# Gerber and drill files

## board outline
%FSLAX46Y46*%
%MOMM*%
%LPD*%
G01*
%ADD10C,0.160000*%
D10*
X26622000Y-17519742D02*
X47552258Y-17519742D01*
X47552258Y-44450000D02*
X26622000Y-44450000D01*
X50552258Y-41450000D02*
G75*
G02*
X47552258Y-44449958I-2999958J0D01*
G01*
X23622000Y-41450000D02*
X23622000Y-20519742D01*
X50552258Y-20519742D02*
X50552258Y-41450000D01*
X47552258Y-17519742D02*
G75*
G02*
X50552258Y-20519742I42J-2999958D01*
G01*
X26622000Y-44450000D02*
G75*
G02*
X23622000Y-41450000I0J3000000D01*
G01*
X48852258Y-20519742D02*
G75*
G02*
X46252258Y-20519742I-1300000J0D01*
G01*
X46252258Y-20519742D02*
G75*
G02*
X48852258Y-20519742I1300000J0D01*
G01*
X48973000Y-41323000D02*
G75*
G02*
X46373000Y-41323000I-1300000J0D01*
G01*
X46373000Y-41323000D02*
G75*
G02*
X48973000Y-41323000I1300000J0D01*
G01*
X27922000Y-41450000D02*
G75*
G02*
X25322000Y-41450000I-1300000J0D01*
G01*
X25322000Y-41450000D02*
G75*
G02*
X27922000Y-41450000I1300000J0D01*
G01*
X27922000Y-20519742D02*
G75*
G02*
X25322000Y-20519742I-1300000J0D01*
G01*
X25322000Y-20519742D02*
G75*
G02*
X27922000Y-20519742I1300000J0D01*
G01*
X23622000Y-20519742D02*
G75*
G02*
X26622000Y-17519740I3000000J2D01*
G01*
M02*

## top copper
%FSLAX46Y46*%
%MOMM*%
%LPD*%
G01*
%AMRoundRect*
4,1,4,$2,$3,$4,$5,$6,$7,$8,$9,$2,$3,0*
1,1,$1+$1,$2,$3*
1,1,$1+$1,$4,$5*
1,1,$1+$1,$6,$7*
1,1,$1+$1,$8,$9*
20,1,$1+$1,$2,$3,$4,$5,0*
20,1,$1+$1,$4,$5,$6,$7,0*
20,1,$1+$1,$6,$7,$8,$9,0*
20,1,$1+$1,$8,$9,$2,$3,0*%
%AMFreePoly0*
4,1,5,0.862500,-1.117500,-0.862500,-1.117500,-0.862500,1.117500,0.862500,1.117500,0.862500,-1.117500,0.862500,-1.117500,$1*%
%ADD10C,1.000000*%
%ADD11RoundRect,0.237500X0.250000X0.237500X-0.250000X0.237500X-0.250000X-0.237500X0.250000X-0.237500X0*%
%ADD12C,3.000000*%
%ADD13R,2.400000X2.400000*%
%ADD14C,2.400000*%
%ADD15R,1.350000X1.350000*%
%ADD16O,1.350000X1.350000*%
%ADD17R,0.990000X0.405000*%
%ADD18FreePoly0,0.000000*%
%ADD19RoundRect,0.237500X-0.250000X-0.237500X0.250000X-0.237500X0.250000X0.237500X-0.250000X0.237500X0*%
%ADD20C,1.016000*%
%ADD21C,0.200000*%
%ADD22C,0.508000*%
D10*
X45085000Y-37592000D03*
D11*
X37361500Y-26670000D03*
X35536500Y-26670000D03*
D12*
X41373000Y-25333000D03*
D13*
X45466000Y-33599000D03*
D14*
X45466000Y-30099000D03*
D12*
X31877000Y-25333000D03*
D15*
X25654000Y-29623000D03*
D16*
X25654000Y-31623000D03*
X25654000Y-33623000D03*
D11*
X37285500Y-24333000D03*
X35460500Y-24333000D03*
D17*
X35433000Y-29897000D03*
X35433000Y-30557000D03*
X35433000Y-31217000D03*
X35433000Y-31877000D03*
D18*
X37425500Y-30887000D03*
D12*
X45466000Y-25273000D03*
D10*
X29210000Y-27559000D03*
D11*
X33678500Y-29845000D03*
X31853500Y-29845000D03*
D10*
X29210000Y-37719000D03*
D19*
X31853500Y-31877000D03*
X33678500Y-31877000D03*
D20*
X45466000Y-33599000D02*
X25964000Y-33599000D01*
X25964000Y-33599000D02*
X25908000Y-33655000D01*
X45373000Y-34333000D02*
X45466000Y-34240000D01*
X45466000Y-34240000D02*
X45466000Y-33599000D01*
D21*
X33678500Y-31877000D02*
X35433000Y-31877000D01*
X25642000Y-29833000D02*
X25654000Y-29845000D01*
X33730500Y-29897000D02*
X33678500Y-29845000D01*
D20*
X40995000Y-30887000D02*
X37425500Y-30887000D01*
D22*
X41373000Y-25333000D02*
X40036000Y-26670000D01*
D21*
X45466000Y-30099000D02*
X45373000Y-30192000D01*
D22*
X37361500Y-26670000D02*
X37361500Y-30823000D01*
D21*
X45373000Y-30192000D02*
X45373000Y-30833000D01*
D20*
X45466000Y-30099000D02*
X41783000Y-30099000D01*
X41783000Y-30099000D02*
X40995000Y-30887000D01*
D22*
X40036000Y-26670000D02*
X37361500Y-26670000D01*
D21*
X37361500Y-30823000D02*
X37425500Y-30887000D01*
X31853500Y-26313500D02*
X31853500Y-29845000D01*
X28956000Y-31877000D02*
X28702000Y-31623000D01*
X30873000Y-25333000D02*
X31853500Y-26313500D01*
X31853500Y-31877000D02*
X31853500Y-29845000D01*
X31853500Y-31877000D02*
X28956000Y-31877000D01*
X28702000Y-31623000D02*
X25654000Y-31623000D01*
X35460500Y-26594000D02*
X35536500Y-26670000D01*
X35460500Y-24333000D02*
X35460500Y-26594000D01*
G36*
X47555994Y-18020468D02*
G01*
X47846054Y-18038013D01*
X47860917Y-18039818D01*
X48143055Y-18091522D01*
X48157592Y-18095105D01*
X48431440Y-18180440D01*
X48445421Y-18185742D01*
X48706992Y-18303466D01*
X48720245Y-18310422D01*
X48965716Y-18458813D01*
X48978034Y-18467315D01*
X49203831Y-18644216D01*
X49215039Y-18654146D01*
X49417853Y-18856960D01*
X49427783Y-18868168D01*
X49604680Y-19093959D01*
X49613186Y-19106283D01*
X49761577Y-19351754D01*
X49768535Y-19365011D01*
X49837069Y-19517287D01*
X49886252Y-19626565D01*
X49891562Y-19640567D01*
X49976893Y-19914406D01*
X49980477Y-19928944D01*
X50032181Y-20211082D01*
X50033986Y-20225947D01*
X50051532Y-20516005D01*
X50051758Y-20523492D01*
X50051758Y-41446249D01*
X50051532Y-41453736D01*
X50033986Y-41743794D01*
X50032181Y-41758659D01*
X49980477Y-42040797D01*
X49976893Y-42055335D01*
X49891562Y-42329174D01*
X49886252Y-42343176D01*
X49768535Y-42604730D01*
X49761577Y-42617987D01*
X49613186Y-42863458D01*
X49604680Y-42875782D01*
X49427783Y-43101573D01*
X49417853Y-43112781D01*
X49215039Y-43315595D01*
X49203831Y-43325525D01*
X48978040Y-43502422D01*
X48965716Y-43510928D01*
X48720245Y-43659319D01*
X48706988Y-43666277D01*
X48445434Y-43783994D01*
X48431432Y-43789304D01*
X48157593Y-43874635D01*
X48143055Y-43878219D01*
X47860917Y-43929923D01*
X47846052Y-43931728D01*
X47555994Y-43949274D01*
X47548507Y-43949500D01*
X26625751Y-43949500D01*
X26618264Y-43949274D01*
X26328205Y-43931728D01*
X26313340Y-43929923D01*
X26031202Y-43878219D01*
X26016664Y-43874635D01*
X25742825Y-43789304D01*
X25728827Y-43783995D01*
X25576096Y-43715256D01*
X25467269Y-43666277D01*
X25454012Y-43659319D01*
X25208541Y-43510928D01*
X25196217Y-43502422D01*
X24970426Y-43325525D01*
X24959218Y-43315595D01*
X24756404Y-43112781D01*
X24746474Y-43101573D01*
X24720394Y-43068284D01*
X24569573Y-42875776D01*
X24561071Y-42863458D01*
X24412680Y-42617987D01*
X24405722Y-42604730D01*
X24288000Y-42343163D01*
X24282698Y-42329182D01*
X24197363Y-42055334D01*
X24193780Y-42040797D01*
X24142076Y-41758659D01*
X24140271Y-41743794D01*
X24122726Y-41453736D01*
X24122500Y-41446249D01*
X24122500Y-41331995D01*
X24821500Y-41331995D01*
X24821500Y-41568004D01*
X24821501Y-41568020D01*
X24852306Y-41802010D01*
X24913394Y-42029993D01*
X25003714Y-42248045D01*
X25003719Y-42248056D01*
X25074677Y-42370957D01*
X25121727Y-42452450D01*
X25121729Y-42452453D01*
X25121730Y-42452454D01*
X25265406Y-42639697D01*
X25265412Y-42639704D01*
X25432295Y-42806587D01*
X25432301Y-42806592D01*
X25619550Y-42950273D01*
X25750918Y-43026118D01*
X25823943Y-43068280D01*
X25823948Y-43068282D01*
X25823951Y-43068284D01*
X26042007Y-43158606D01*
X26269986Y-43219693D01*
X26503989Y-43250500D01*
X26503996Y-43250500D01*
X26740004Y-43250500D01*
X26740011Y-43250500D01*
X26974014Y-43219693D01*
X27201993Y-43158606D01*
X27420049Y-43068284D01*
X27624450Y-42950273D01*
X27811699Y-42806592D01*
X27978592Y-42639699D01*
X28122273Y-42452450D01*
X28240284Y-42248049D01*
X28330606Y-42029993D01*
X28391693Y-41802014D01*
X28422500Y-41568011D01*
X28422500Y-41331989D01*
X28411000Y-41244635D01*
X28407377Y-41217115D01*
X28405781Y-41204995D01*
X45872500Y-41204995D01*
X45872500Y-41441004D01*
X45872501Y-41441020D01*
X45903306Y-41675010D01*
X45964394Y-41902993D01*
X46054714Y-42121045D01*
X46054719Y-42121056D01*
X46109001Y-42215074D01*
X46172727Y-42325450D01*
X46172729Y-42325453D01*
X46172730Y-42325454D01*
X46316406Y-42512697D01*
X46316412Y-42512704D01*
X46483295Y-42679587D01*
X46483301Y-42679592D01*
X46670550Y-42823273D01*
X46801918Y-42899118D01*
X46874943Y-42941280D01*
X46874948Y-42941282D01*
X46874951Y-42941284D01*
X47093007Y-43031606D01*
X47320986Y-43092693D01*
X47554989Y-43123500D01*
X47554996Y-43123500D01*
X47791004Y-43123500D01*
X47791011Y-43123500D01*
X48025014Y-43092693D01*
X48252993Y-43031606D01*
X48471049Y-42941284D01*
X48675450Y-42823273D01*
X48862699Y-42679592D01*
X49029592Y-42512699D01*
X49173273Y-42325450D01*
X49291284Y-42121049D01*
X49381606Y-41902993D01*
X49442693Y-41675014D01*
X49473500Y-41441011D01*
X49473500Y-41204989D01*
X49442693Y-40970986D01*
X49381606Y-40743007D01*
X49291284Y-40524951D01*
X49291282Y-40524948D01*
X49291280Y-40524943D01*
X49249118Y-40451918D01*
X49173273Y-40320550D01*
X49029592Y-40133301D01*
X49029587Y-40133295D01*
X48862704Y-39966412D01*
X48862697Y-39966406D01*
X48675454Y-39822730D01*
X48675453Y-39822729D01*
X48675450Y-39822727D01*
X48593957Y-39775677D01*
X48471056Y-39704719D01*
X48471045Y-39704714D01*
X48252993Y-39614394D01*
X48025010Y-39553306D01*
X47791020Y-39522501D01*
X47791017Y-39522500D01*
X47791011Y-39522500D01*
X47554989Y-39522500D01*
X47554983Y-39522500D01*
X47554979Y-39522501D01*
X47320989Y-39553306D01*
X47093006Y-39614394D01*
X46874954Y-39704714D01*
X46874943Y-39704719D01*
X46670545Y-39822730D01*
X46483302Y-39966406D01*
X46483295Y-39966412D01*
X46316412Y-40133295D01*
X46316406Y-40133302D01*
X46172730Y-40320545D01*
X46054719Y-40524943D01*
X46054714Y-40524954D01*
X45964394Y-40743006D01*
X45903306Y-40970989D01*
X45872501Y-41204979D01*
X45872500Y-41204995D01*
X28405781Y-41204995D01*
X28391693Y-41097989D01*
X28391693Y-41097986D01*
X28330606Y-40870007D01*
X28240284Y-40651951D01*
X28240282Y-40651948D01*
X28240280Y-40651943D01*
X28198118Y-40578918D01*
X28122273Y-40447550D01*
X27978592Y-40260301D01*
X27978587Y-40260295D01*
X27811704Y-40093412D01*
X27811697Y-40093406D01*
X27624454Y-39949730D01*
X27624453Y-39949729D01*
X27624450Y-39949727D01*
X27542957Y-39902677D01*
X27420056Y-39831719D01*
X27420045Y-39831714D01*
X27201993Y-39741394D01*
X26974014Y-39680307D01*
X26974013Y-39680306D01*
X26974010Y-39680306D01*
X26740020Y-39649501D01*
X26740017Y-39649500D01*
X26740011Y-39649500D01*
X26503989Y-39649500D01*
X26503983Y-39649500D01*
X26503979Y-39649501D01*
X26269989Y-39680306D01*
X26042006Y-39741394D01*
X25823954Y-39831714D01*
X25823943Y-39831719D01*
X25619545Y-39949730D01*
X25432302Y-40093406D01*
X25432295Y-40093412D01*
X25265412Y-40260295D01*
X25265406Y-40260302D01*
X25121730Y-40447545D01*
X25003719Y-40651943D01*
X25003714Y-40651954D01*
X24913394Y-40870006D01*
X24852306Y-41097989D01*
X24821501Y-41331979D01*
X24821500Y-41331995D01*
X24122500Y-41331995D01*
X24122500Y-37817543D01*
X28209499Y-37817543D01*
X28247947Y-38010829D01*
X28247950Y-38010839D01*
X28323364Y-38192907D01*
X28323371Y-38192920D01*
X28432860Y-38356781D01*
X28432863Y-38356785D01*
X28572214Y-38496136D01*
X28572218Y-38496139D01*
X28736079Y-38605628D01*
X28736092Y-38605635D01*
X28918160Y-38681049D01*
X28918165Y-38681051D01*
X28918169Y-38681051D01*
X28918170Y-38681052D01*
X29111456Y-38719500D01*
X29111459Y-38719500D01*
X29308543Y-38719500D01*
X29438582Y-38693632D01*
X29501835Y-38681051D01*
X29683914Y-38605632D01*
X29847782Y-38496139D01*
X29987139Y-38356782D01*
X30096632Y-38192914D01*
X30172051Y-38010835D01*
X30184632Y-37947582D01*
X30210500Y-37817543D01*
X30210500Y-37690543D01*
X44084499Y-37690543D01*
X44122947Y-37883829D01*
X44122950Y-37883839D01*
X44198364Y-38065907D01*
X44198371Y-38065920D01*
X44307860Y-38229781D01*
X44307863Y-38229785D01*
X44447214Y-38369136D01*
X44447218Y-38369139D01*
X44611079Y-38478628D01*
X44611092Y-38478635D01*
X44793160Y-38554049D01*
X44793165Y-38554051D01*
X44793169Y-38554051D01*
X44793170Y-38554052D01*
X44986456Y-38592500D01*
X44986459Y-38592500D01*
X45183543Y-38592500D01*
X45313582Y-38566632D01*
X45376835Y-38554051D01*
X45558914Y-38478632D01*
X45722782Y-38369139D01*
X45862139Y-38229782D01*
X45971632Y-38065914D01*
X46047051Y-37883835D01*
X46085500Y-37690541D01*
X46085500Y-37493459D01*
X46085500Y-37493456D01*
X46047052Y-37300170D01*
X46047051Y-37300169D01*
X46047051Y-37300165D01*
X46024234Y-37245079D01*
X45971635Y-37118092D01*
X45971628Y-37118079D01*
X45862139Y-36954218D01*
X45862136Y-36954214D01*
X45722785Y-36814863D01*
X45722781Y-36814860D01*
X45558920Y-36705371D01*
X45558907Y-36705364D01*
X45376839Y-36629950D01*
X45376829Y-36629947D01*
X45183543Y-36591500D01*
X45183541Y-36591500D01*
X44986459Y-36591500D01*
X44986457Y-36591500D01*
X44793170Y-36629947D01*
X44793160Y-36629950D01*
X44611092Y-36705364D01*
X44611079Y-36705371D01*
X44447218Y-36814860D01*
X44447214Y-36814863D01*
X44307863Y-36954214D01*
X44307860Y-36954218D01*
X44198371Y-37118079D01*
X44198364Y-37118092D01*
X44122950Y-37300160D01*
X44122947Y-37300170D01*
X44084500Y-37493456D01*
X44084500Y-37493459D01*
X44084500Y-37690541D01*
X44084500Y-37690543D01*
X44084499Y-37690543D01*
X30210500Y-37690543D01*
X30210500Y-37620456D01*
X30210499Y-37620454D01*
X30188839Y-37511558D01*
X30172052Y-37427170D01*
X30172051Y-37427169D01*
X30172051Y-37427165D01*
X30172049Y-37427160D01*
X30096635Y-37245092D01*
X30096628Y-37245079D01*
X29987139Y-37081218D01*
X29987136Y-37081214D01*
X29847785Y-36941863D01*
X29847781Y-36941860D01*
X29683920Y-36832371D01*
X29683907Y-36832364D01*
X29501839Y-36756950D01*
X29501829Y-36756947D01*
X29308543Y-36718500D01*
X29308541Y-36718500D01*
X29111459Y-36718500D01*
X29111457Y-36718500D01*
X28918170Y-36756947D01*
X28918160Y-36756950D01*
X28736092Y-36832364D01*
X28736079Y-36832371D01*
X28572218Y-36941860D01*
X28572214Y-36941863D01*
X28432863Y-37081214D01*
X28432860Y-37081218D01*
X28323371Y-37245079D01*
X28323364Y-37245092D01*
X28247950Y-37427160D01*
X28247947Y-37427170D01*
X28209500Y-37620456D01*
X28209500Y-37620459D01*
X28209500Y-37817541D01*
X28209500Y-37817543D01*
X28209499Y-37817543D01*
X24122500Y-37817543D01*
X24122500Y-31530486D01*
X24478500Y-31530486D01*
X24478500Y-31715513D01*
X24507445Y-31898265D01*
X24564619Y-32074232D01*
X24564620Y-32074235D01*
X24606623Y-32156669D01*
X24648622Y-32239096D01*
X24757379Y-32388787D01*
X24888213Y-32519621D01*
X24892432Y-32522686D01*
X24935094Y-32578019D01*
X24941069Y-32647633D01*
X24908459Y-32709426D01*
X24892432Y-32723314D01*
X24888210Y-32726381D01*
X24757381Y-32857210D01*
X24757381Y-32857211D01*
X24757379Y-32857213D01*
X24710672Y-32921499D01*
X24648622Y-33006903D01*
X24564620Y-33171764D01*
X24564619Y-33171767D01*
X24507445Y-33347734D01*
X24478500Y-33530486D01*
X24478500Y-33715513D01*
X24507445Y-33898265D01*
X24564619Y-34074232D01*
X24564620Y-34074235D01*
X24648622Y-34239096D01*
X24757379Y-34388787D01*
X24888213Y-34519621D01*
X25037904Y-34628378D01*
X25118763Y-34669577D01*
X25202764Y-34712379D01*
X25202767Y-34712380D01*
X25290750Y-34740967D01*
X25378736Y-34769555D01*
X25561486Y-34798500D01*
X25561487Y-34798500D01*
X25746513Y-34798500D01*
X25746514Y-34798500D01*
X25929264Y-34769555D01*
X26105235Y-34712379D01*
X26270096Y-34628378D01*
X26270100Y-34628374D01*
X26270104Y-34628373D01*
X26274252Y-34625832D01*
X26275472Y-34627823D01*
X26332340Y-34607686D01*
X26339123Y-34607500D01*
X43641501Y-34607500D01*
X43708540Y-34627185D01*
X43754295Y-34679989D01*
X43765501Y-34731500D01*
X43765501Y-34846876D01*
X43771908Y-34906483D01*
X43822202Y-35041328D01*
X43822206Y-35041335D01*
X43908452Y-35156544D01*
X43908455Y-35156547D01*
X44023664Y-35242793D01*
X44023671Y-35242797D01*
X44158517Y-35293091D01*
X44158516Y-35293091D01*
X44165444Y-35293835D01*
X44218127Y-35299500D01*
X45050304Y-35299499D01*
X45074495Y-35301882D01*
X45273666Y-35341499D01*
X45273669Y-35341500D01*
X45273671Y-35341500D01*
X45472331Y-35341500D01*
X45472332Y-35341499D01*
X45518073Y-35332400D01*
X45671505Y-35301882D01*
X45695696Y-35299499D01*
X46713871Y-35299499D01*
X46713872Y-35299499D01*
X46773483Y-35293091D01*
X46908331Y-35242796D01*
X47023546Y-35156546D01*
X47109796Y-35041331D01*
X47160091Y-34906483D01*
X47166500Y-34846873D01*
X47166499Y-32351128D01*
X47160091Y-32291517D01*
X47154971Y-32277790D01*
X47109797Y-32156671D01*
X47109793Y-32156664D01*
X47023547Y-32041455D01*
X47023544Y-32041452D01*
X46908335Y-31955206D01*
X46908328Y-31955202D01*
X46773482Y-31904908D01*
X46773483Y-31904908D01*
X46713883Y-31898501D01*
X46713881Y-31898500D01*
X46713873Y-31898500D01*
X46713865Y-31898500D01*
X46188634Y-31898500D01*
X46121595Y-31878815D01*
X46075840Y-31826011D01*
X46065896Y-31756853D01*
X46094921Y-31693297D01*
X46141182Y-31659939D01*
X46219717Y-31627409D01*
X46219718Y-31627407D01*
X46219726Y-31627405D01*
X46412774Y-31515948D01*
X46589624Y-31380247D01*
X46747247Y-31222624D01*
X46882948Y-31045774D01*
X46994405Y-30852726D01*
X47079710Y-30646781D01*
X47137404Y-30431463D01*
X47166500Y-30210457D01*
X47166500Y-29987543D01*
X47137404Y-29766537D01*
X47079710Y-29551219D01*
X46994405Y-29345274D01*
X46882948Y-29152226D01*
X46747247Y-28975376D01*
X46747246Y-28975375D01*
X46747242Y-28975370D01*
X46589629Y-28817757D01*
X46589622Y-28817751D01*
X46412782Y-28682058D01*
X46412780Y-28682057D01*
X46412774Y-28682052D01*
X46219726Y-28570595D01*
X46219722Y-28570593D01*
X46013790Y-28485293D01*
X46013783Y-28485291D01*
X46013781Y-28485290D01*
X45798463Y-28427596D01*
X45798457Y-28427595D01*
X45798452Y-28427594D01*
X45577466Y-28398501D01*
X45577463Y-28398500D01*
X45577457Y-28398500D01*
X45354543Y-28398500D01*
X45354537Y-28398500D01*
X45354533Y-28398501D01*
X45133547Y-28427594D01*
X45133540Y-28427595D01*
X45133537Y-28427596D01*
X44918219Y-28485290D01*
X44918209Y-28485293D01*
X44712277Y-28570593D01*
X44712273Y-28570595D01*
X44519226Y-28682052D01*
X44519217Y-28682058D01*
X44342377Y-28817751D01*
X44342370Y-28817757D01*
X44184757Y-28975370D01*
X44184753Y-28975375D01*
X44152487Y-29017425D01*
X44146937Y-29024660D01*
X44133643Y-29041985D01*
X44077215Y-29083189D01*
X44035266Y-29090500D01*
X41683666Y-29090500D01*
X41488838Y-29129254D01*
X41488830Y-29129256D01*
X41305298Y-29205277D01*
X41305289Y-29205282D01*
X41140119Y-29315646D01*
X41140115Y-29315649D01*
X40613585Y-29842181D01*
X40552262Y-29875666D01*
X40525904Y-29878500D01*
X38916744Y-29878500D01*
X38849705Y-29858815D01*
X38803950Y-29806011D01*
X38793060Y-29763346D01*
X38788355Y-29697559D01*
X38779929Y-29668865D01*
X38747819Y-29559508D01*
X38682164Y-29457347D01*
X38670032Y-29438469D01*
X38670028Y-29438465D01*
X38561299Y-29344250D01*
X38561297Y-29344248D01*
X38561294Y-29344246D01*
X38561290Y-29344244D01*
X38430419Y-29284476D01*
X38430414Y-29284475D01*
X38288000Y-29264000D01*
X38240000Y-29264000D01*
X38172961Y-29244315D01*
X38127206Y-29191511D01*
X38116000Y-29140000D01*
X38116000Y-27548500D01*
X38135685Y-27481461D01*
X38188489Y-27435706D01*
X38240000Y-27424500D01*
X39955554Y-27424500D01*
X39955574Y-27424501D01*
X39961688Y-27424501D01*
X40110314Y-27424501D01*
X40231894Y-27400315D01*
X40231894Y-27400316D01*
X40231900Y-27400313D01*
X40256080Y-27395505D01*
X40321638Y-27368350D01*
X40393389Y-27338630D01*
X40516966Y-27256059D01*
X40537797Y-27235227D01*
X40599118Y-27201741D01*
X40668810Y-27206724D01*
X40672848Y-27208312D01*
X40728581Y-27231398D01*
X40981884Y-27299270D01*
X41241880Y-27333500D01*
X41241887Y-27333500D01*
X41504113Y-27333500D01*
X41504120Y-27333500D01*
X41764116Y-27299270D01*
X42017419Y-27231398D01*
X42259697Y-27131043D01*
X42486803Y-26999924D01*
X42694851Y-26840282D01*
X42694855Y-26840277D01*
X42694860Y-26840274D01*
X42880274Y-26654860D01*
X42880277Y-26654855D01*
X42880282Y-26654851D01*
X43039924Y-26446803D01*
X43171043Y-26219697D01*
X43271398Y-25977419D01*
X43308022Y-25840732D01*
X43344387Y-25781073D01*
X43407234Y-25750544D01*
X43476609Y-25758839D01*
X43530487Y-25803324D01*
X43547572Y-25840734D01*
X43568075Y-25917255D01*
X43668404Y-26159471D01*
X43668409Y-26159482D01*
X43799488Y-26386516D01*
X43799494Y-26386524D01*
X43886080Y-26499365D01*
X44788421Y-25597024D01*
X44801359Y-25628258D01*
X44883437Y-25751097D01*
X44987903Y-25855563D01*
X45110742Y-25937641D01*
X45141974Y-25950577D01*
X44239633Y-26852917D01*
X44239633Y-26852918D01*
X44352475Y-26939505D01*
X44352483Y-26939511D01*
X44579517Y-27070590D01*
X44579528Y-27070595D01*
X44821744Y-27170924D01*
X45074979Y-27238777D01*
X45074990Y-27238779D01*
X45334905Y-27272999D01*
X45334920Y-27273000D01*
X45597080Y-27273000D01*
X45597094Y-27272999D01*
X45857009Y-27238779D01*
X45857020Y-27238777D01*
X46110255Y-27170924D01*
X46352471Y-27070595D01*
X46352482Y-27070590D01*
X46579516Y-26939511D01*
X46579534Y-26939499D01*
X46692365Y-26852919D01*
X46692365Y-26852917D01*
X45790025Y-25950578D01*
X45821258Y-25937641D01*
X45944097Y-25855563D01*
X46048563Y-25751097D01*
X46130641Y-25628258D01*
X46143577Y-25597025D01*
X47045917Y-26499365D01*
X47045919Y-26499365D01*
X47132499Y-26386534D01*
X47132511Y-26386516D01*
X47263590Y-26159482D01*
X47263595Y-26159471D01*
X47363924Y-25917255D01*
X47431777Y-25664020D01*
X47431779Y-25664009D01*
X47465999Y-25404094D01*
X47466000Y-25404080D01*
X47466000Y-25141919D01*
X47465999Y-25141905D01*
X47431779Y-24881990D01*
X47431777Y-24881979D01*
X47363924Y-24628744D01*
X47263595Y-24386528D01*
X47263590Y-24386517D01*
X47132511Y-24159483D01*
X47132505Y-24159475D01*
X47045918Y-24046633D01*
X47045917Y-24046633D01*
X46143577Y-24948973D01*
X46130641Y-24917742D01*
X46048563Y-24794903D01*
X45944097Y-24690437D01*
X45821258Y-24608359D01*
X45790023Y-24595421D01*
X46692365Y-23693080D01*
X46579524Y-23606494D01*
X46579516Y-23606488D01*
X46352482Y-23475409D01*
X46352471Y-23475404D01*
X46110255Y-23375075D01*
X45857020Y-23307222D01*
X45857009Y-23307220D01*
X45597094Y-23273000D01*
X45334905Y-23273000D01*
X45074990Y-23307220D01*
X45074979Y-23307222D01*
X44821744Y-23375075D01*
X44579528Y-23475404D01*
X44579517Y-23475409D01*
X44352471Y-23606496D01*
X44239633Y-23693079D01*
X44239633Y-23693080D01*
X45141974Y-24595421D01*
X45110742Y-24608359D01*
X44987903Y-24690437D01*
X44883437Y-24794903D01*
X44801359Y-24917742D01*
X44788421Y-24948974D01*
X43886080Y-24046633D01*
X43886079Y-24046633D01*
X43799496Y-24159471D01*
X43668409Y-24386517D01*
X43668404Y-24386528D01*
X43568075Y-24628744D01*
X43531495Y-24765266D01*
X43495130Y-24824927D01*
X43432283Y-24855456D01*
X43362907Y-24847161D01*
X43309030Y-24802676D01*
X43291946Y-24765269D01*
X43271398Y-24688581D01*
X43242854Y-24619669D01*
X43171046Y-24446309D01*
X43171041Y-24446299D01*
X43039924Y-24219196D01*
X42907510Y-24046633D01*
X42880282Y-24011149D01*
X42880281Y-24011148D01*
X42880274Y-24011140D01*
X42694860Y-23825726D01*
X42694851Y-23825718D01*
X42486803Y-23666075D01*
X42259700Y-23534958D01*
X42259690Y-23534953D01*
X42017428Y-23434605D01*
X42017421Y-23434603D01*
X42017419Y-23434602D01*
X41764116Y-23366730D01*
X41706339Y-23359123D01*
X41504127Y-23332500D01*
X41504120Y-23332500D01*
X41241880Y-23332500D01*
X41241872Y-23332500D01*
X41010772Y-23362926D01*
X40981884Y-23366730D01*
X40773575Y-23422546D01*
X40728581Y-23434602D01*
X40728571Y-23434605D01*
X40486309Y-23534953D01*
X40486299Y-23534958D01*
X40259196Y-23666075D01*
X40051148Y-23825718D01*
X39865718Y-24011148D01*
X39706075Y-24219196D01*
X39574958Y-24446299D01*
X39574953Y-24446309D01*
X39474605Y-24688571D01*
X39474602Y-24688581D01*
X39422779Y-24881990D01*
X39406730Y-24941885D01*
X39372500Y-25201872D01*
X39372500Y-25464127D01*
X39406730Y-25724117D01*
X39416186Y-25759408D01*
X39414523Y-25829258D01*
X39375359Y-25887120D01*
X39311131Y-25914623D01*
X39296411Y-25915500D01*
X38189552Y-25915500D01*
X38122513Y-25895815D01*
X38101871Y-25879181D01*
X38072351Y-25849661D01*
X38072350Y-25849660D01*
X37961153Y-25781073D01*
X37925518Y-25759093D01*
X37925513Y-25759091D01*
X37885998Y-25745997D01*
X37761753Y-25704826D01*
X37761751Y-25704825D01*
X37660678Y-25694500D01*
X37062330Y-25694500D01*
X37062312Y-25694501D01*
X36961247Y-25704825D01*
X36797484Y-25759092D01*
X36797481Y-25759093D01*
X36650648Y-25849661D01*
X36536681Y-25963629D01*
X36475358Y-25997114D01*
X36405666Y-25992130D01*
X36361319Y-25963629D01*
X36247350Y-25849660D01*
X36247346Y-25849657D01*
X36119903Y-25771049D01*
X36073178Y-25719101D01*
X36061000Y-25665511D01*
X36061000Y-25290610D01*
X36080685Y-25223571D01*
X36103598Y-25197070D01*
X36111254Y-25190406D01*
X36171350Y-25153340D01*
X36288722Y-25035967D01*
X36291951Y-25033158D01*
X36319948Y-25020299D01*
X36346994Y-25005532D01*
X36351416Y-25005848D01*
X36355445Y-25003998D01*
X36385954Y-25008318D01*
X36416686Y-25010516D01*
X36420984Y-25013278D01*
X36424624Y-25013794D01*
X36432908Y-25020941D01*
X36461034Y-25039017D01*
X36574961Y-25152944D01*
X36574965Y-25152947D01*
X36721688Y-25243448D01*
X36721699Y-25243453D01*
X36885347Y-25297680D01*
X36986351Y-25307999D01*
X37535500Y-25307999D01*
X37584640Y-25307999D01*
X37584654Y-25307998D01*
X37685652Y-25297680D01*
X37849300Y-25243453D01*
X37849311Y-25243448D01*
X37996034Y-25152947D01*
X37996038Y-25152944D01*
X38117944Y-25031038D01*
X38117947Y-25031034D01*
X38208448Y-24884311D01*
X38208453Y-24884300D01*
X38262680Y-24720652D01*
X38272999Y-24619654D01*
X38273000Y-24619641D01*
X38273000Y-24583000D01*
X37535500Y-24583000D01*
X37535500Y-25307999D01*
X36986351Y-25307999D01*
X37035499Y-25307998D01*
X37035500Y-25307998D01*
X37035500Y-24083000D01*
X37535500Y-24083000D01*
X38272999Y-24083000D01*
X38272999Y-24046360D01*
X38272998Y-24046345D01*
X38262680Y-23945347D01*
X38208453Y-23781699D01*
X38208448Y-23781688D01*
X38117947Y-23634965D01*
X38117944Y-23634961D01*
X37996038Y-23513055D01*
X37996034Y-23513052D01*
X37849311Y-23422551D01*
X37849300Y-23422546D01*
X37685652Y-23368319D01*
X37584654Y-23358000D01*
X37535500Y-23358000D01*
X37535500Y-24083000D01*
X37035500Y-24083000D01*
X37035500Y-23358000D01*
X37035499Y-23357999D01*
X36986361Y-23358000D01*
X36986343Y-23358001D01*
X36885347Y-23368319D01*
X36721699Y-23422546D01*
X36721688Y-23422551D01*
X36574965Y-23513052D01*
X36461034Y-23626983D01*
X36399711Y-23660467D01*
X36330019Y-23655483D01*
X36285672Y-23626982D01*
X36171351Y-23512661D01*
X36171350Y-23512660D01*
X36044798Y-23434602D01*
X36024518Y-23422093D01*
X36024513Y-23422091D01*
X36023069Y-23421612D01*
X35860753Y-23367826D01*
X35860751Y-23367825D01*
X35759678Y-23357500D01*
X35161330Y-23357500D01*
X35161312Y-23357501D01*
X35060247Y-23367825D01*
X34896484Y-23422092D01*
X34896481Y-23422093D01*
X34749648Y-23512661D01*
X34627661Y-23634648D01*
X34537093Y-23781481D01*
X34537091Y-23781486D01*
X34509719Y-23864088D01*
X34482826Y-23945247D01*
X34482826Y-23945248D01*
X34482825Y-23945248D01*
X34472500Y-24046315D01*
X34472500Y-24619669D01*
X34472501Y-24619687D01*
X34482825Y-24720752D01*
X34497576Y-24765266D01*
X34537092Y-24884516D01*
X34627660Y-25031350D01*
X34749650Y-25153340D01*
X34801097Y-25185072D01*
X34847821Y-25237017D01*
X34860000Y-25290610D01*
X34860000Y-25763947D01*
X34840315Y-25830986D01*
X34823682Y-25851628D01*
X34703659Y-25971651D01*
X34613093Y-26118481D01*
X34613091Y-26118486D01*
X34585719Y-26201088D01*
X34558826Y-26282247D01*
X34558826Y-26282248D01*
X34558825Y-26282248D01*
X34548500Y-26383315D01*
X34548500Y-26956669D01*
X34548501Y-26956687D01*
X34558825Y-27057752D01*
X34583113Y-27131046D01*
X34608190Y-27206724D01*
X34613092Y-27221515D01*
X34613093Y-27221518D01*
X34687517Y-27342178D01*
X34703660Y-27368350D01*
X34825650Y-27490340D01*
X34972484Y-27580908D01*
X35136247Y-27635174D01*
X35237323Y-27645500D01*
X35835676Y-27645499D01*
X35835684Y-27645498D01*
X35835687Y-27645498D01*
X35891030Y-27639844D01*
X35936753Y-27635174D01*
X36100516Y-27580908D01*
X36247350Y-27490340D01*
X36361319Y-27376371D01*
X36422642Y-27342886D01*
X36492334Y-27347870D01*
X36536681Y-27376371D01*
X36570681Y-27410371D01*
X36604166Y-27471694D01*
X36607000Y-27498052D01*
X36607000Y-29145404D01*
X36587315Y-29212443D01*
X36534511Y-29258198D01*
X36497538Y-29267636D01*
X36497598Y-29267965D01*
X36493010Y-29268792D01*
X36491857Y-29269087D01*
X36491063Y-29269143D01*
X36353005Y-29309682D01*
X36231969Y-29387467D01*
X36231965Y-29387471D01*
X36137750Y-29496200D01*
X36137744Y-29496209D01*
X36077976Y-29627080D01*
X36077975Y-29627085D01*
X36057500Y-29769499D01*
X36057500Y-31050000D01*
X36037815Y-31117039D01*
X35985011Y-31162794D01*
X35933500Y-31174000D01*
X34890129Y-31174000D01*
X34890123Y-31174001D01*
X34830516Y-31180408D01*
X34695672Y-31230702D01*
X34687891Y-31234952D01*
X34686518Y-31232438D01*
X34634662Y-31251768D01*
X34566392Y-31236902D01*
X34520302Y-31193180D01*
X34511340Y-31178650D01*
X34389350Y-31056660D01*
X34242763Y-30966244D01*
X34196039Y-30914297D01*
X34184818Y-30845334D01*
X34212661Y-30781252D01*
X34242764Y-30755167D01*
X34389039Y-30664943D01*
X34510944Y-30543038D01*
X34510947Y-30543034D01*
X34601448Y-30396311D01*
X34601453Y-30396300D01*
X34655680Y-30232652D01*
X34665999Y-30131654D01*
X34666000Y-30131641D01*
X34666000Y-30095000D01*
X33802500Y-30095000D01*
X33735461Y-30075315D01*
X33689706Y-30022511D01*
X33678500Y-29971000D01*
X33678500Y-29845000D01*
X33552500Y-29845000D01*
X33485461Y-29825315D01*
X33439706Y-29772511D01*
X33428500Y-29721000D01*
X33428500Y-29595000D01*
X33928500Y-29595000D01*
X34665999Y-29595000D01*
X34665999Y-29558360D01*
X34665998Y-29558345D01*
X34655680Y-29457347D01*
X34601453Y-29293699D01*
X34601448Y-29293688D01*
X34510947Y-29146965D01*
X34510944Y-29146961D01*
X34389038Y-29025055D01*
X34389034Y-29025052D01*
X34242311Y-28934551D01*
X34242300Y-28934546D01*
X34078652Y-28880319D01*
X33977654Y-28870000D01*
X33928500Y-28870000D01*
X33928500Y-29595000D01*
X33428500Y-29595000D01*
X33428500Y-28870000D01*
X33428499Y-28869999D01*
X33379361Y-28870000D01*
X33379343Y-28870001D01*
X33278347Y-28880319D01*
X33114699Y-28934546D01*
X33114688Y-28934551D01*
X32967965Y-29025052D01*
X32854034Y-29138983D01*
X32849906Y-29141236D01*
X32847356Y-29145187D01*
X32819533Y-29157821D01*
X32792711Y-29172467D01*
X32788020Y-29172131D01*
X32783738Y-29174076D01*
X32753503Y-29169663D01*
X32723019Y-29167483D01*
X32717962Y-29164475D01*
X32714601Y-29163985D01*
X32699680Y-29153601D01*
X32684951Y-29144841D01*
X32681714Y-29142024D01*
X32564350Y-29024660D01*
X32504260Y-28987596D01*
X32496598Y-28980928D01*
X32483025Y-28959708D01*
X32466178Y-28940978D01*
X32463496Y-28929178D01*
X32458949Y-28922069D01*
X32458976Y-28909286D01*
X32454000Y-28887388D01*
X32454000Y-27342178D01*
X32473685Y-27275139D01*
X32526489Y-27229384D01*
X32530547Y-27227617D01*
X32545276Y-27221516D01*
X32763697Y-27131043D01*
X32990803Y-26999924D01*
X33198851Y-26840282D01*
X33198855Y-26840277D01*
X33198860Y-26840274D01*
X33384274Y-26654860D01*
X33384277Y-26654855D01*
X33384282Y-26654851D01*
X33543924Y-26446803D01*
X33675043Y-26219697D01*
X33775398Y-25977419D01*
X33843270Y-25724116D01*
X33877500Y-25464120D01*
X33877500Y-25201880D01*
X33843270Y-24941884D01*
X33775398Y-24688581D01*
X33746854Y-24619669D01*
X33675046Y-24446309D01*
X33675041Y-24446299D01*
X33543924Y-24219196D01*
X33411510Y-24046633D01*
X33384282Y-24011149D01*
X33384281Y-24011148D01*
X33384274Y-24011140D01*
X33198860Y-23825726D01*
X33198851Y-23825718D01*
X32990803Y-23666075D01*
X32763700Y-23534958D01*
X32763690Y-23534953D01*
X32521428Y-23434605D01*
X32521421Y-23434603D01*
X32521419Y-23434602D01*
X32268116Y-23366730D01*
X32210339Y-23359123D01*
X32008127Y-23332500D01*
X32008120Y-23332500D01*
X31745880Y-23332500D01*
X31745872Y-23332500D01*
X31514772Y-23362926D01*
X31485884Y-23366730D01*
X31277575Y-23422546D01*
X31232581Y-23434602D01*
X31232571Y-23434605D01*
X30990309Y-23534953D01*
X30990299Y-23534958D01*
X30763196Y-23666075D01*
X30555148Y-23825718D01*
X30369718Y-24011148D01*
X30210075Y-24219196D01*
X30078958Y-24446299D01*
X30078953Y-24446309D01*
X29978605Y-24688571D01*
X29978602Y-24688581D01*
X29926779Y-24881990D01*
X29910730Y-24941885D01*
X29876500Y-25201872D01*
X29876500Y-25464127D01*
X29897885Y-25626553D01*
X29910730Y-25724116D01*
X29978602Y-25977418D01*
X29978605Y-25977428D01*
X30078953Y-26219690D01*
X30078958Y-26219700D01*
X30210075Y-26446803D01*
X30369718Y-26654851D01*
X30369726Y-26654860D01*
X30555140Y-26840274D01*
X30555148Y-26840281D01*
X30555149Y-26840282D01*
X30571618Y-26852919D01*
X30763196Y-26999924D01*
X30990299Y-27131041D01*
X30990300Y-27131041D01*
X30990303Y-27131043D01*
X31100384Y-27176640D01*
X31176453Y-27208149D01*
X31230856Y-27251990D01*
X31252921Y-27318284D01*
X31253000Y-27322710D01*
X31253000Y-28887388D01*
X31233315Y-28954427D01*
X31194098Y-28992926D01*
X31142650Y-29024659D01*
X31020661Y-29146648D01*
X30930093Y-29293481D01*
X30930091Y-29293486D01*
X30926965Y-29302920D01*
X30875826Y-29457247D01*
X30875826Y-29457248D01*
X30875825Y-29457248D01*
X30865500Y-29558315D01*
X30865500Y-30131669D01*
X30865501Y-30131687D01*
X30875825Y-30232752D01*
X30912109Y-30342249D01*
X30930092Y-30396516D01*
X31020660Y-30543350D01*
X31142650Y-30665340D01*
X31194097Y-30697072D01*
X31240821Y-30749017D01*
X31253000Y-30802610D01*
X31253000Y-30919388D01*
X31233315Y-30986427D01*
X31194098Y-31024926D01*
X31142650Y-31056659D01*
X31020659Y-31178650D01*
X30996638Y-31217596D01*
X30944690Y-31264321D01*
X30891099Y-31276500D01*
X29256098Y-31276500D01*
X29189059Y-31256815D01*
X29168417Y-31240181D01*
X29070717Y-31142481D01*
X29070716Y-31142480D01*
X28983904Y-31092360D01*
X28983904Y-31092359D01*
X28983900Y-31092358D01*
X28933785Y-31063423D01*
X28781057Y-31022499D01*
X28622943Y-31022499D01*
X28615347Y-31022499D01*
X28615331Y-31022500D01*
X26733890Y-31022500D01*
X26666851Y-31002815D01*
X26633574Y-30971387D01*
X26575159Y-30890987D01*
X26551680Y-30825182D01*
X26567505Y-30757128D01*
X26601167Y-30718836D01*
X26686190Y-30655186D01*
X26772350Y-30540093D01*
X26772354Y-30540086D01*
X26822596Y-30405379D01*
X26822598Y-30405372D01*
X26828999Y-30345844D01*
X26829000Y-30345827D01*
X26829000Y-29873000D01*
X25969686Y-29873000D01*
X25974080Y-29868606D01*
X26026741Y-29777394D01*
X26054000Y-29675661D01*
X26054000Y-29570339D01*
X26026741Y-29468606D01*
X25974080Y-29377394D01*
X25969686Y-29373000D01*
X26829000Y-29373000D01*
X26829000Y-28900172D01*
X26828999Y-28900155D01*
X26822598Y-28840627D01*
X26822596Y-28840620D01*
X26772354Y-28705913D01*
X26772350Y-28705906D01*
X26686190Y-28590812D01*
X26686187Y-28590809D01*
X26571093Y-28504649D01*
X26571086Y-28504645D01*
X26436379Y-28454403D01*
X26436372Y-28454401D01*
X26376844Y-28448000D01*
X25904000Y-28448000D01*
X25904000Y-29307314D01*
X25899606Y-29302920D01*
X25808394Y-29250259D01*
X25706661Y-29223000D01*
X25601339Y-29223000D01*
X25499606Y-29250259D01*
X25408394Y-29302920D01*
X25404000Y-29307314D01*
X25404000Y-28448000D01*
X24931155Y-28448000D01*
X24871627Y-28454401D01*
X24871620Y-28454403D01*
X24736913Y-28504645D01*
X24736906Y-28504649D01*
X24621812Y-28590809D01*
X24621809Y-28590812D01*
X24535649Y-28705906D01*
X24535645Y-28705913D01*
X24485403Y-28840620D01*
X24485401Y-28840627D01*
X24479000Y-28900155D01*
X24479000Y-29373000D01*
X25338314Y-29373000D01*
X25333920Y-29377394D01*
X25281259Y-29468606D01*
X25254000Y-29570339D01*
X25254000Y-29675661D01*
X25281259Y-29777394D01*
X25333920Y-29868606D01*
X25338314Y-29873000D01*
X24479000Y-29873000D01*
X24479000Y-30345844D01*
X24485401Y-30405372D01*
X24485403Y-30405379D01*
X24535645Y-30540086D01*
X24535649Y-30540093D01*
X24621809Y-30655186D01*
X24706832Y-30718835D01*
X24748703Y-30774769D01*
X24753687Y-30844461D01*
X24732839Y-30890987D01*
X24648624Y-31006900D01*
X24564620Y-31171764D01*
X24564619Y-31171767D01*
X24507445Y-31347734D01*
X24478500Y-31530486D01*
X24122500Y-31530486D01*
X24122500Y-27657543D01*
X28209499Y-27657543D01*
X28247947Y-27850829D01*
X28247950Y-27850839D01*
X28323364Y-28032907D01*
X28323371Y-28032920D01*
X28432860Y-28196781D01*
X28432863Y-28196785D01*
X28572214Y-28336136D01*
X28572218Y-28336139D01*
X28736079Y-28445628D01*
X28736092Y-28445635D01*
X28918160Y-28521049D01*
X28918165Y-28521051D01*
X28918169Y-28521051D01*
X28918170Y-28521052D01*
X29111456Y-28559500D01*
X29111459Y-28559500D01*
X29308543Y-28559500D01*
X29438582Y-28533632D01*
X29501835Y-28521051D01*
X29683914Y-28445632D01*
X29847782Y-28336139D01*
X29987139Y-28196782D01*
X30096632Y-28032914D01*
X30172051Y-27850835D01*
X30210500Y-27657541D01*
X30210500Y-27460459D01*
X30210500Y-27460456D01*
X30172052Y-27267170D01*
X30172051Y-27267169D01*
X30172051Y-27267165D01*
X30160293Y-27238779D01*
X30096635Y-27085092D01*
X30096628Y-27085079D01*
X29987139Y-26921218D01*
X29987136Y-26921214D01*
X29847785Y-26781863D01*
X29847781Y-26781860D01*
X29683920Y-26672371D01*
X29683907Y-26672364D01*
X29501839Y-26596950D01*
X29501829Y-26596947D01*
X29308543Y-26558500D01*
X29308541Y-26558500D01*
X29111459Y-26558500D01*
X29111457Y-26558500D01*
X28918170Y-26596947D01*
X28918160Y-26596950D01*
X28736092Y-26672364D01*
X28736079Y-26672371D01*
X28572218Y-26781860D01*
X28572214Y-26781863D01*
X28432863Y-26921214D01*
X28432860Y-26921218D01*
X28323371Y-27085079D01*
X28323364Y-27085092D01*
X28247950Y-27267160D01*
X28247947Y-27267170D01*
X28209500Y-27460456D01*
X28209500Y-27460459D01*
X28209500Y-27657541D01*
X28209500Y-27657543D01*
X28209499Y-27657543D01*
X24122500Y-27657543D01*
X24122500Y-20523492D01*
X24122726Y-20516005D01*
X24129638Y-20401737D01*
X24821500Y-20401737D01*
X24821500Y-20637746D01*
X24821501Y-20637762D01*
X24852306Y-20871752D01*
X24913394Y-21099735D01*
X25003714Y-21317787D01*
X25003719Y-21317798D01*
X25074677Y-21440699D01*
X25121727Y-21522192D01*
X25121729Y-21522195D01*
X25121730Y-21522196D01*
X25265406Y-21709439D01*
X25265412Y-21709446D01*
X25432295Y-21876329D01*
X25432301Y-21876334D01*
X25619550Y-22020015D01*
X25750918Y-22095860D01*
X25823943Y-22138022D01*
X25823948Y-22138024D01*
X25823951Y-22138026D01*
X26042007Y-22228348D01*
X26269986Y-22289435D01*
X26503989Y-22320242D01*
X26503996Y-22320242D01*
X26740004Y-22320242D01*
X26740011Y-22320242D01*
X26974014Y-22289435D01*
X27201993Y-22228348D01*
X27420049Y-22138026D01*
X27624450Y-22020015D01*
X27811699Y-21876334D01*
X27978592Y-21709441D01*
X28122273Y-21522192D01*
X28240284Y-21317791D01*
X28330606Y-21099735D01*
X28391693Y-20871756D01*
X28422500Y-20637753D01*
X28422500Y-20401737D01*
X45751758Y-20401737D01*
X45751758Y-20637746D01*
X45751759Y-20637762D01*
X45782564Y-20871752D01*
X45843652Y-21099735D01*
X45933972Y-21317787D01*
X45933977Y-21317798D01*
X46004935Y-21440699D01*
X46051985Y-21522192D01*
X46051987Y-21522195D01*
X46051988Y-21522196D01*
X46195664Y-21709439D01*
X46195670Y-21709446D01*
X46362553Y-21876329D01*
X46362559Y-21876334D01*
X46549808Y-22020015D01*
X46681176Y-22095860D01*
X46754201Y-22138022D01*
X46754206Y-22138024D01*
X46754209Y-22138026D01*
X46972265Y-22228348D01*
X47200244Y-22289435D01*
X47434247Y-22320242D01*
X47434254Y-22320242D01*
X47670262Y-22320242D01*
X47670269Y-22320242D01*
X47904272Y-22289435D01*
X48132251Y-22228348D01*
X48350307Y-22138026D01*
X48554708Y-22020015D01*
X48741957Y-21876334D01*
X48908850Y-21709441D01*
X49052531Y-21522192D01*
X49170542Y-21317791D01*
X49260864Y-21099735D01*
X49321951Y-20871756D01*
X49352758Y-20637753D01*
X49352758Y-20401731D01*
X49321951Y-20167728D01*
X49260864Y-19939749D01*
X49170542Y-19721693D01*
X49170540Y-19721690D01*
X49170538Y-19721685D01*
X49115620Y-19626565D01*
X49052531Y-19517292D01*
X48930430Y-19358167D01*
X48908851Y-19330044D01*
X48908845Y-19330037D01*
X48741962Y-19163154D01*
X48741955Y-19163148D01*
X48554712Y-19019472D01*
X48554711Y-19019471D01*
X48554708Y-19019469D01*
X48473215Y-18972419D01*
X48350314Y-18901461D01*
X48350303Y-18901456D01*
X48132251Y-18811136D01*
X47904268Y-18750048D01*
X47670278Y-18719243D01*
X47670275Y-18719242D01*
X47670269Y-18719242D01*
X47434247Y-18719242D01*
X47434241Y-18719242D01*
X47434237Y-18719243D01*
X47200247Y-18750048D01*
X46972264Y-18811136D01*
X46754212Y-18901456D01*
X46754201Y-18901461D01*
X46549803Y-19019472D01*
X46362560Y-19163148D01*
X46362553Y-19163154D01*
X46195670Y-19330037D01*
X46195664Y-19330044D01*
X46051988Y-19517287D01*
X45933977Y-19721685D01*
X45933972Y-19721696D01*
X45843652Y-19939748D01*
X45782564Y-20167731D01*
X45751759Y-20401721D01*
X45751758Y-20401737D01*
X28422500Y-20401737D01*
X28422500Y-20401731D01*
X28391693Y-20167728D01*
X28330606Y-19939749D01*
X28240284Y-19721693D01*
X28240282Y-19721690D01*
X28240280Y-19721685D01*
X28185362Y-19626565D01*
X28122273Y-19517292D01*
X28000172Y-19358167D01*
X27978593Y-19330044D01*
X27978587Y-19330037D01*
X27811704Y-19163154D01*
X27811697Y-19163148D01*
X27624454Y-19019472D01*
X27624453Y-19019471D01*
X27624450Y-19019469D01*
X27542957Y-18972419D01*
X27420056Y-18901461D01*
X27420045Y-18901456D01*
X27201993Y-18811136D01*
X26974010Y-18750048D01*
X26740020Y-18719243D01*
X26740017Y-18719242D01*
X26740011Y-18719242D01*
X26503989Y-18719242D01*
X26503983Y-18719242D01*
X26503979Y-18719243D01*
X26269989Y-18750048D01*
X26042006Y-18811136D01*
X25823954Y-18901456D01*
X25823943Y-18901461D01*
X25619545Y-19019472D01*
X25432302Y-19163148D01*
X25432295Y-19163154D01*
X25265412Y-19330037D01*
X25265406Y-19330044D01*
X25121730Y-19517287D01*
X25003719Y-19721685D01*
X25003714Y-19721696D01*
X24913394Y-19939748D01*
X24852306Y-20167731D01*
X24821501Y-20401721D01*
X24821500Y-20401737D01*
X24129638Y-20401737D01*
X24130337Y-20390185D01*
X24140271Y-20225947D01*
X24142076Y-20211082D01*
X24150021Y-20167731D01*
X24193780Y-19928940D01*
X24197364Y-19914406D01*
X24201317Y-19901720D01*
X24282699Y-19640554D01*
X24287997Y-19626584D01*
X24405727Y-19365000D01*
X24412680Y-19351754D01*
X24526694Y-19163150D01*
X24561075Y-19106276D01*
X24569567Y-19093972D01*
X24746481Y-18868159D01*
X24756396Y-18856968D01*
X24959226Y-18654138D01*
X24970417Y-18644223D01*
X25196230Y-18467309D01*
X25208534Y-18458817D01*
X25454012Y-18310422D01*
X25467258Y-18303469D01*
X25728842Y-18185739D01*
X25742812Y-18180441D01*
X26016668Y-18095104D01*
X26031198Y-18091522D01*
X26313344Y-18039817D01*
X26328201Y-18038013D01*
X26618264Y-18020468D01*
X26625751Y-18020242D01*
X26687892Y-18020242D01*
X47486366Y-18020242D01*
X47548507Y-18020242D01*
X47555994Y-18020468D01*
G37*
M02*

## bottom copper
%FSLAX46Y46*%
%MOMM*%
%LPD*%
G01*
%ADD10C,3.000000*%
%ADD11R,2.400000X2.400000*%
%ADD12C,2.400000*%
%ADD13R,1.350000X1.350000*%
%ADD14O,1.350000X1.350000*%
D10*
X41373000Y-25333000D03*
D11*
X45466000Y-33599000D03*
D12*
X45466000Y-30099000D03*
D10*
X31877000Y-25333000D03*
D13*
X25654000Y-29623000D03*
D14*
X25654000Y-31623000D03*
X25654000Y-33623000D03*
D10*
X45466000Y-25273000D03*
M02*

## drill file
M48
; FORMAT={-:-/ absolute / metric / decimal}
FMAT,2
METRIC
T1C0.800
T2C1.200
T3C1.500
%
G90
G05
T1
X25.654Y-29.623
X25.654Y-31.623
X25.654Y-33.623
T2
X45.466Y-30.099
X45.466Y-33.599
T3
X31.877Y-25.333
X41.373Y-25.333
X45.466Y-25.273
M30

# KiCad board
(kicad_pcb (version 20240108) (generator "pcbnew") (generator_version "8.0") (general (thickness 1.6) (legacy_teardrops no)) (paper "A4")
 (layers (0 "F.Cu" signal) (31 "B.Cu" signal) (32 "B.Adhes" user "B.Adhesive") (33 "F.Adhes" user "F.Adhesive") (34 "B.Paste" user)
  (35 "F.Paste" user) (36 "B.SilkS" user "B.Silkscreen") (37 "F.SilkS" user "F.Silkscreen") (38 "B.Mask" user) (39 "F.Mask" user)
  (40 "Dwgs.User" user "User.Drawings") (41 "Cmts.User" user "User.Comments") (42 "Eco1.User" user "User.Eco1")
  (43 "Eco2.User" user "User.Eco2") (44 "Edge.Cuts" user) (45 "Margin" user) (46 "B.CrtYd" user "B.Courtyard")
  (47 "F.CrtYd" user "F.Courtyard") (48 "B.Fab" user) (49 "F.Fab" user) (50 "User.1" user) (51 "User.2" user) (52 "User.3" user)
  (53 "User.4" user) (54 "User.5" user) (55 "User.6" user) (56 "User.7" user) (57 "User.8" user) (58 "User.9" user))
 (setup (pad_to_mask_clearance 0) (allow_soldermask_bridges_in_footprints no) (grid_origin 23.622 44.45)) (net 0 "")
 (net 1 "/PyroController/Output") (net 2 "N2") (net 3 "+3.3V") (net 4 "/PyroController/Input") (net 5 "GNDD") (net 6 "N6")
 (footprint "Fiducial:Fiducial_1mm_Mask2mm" (layer "F.Cu") (at 45.085 37.592)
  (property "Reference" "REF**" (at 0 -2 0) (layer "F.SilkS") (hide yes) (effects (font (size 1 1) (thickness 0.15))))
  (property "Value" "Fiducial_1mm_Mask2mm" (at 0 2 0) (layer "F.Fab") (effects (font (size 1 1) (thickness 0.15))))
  (pad "" smd circle (at 0 0) (size 1 1) (layers "F.Cu" "F.Mask") (solder_mask_margin 0.5) (clearance 0.5)))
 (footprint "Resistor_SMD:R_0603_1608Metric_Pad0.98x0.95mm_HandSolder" (layer "F.Cu") (at 36.449 26.67 180)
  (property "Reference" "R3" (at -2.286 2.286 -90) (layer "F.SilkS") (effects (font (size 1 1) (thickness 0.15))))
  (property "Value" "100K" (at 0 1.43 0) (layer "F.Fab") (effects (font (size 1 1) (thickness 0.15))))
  (pad "1" smd roundrect (at -0.9125 0 180) (size 0.975 0.95) (layers "F.Cu" "F.Paste" "F.Mask") (roundrect_rratio 0.25)
   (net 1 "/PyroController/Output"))
  (pad "2" smd roundrect (at 0.9125 0 180) (size 0.975 0.95) (layers "F.Cu" "F.Paste" "F.Mask") (roundrect_rratio 0.25) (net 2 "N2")))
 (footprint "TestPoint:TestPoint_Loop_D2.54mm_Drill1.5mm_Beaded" (layer "F.Cu") (at 41.373 25.333)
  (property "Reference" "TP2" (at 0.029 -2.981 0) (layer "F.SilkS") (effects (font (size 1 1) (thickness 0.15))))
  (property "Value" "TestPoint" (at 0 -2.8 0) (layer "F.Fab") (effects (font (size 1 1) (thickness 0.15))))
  (pad "1" thru_hole circle (at 0 0) (size 3 3) (drill 1.5) (layers "*.Cu" "*.Mask") (remove_unused_layers no)
   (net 1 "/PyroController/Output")))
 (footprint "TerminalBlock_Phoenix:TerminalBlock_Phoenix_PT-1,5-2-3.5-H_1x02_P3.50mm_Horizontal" (layer "F.Cu") (at 45.466 33.599 90)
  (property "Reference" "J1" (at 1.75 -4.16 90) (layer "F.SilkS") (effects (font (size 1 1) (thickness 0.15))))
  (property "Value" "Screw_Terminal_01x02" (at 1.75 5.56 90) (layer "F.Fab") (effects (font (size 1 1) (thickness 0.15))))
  (pad "1" thru_hole rect (at 0 0 90) (size 2.4 2.4) (drill 1.2) (layers "*.Cu" "*.Mask") (remove_unused_layers no) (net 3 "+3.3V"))
  (pad "2" thru_hole circle (at 3.5 0 90) (size 2.4 2.4) (drill 1.2) (layers "*.Cu" "*.Mask") (remove_unused_layers no)
   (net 1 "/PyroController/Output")))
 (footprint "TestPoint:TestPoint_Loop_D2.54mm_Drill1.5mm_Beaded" (layer "F.Cu") (at 31.877 25.333)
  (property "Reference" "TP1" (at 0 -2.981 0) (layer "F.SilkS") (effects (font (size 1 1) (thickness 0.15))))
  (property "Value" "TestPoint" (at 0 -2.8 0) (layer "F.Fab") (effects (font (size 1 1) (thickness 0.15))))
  (pad "1" thru_hole circle (at 0 0) (size 3 3) (drill 1.5) (layers "*.Cu" "*.Mask") (remove_unused_layers no)
   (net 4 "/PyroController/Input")))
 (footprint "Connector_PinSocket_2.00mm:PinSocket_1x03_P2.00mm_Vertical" (layer "F.Cu") (at 25.654 29.623)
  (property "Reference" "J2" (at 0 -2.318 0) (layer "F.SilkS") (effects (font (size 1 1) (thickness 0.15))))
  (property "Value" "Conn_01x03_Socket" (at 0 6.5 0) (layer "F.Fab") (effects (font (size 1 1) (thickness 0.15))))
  (pad "1" thru_hole rect (at 0 0) (size 1.35 1.35) (drill 0.8) (layers "*.Cu" "*.Mask") (remove_unused_layers no) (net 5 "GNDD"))
  (pad "2" thru_hole oval (at 0 2) (size 1.35 1.35) (drill 0.8) (layers "*.Cu" "*.Mask") (remove_unused_layers no)
   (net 4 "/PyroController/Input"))
  (pad "3" thru_hole oval (at 0 4) (size 1.35 1.35) (drill 0.8) (layers "*.Cu" "*.Mask") (remove_unused_layers no) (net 3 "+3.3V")))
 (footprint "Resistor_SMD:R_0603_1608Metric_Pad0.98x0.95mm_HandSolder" (layer "F.Cu") (at 36.373 24.333 180)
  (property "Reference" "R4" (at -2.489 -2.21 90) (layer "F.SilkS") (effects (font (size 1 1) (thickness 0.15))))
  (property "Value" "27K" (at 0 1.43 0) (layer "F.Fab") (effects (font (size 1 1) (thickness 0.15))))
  (pad "1" smd roundrect (at -0.9125 0 180) (size 0.975 0.95) (layers "F.Cu" "F.Paste" "F.Mask") (roundrect_rratio 0.25) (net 5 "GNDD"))
  (pad "2" smd roundrect (at 0.9125 0 180) (size 0.975 0.95) (layers "F.Cu" "F.Paste" "F.Mask") (roundrect_rratio 0.25) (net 2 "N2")))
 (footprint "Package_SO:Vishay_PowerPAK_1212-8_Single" (layer "F.Cu") (at 36.868 30.887)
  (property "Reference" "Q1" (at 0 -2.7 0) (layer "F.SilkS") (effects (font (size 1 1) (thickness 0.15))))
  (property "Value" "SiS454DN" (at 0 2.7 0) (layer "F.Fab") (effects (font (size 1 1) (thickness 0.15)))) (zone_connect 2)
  (pad "1" smd rect (at -1.435 -0.99) (size 0.99 0.405) (layers "F.Cu" "F.Paste" "F.Mask") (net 5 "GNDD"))
  (pad "2" smd rect (at -1.435 -0.33) (size 0.99 0.405) (layers "F.Cu" "F.Paste" "F.Mask") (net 5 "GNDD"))
  (pad "3" smd rect (at -1.435 0.33) (size 0.99 0.405) (layers "F.Cu" "F.Paste" "F.Mask") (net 5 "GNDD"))
  (pad "4" smd rect (at -1.435 0.99) (size 0.99 0.405) (layers "F.Cu" "F.Paste" "F.Mask") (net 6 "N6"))
  (pad "5" smd custom (at 0.5575 0) (size 1.725 2.235) (layers "F.Cu" "F.Paste" "F.Mask") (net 1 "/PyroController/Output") (zone_connect 2)
   (thermal_bridge_angle 45) (options (clearance outline) (anchor rect)) (primitives)))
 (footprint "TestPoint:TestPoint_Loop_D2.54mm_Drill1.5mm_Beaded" (layer "F.Cu") (at 45.466 25.273)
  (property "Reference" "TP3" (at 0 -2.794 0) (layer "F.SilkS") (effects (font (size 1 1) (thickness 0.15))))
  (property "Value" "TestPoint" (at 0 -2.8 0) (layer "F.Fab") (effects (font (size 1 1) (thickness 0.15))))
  (pad "1" thru_hole circle (at 0 0) (size 3 3) (drill 1.5) (layers "*.Cu" "*.Mask") (remove_unused_layers no) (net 5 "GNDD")))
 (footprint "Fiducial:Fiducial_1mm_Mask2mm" (layer "F.Cu") (at 29.21 27.559)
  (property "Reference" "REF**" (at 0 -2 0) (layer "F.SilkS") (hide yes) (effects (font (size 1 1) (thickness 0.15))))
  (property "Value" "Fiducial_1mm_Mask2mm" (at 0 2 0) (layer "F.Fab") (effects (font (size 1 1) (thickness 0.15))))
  (pad "" smd circle (at 0 0) (size 1 1) (layers "F.Cu" "F.Mask") (solder_mask_margin 0.5) (clearance 0.5)))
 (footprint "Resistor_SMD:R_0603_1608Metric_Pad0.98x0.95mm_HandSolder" (layer "F.Cu") (at 32.766 29.845 180)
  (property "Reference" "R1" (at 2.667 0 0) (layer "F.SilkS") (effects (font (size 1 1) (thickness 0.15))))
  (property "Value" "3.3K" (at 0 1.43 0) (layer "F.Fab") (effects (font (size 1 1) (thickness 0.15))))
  (pad "1" smd roundrect (at -0.9125 0 180) (size 0.975 0.95) (layers "F.Cu" "F.Paste" "F.Mask") (roundrect_rratio 0.25) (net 5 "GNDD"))
  (pad "2" smd roundrect (at 0.9125 0 180) (size 0.975 0.95) (layers "F.Cu" "F.Paste" "F.Mask") (roundrect_rratio 0.25)
   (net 4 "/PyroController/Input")))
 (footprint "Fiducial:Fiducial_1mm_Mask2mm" (layer "F.Cu") (at 29.21 37.719)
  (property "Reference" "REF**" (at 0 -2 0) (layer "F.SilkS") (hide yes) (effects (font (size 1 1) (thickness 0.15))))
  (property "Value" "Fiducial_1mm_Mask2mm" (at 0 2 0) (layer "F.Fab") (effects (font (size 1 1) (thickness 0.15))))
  (pad "" smd circle (at 0 0) (size 1 1) (layers "F.Cu" "F.Mask") (solder_mask_margin 0.5) (clearance 0.5)))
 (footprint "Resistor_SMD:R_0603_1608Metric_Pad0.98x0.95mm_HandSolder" (layer "F.Cu") (at 32.766 31.877)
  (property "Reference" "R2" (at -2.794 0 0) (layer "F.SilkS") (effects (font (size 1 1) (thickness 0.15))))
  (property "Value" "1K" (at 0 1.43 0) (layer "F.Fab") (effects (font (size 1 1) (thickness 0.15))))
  (pad "1" smd roundrect (at -0.9125 0) (size 0.975 0.95) (layers "F.Cu" "F.Paste" "F.Mask") (roundrect_rratio 0.25)
   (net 4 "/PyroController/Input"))
  (pad "2" smd roundrect (at 0.9125 0) (size 0.975 0.95) (layers "F.Cu" "F.Paste" "F.Mask") (roundrect_rratio 0.25) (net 6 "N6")))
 (gr_line (start 26.622 17.519742) (end 47.552258 17.519742) (stroke (width 0.16) (type solid)) (layer "Edge.Cuts"))
 (gr_line (start 47.552258 44.45) (end 26.622 44.45) (stroke (width 0.16) (type solid)) (layer "Edge.Cuts"))
 (gr_arc (start 50.552258 41.45) (mid 49.673578 43.57132) (end 47.552258 44.45) (stroke (width 0.16) (type solid)) (layer "Edge.Cuts"))
 (gr_line (start 23.622 41.45) (end 23.622 20.519742) (stroke (width 0.16) (type solid)) (layer "Edge.Cuts"))
 (gr_line (start 50.552258 20.519742) (end 50.552258 41.45) (stroke (width 0.16) (type solid)) (layer "Edge.Cuts"))
 (gr_arc (start 47.552258 17.519742) (mid 49.673578 18.398422) (end 50.552258 20.519742) (stroke (width 0.16) (type solid))
  (layer "Edge.Cuts"))
 (gr_arc (start 26.622 44.45) (mid 24.50068 43.57132) (end 23.622 41.45) (stroke (width 0.16) (type solid)) (layer "Edge.Cuts"))
 (gr_circle (center 47.552258 20.519742) (end 46.252258 20.519742) (stroke (width 0.16) (type solid)) (fill none) (layer "Edge.Cuts"))
 (gr_circle (center 47.673 41.323) (end 46.373 41.323) (stroke (width 0.16) (type solid)) (fill none) (layer "Edge.Cuts"))
 (gr_circle (center 26.622 41.45) (end 25.322 41.45) (stroke (width 0.16) (type solid)) (fill none) (layer "Edge.Cuts"))
 (gr_circle (center 26.622 20.519742) (end 25.322 20.519742) (stroke (width 0.16) (type solid)) (fill none) (layer "Edge.Cuts"))
 (gr_arc (start 23.622 20.519742) (mid 24.50068 18.398422) (end 26.622 17.519742) (stroke (width 0.16) (type solid)) (layer "Edge.Cuts"))
 (segment (start 45.466 33.599) (end 25.964 33.599) (width 1.016) (layer "F.Cu") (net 3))
 (segment (start 25.964 33.599) (end 25.908 33.655) (width 1.016) (layer "F.Cu") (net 3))
 (segment (start 45.373 34.333) (end 45.466 34.24) (width 1.016) (layer "F.Cu") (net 3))
 (segment (start 45.466 34.24) (end 45.466 33.599) (width 1.016) (layer "F.Cu") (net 3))
 (segment (start 33.6785 31.877) (end 35.433 31.877) (width 0.2) (layer "F.Cu") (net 6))
 (segment (start 25.642 29.833) (end 25.654 29.845) (width 0.2) (layer "F.Cu") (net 5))
 (segment (start 33.7305 29.897) (end 33.6785 29.845) (width 0.2) (layer "F.Cu") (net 5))
 (segment (start 40.995 30.887) (end 37.4255 30.887) (width 1.016) (layer "F.Cu") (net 1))
 (segment (start 41.373 25.333) (end 40.036 26.67) (width 0.508) (layer "F.Cu") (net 1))
 (segment (start 45.466 30.099) (end 45.373 30.192) (width 0.2) (layer "F.Cu") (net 1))
 (segment (start 37.3615 26.67) (end 37.3615 30.823) (width 0.508) (layer "F.Cu") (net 1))
 (segment (start 45.373 30.192) (end 45.373 30.833) (width 0.2) (layer "F.Cu") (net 1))
 (segment (start 45.466 30.099) (end 41.783 30.099) (width 1.016) (layer "F.Cu") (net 1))
 (segment (start 41.783 30.099) (end 40.995 30.887) (width 1.016) (layer "F.Cu") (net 1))
 (segment (start 40.036 26.67) (end 37.3615 26.67) (width 0.508) (layer "F.Cu") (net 1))
 (segment (start 37.3615 30.823) (end 37.4255 30.887) (width 0.2) (layer "F.Cu") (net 1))
 (segment (start 31.8535 26.3135) (end 31.8535 29.845) (width 0.2) (layer "F.Cu") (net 4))
 (segment (start 28.956 31.877) (end 28.702 31.623) (width 0.2) (layer "F.Cu") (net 4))
 (segment (start 30.873 25.333) (end 31.8535 26.3135) (width 0.2) (layer "F.Cu") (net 4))
 (segment (start 31.8535 31.877) (end 31.8535 29.845) (width 0.2) (layer "F.Cu") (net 4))
 (segment (start 31.8535 31.877) (end 28.956 31.877) (width 0.2) (layer "F.Cu") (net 4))
 (segment (start 28.702 31.623) (end 25.654 31.623) (width 0.2) (layer "F.Cu") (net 4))
 (segment (start 35.4605 26.594) (end 35.5365 26.67) (width 0.2) (layer "F.Cu") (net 2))
 (segment (start 35.4605 24.333) (end 35.4605 26.594) (width 0.2) (layer "F.Cu") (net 2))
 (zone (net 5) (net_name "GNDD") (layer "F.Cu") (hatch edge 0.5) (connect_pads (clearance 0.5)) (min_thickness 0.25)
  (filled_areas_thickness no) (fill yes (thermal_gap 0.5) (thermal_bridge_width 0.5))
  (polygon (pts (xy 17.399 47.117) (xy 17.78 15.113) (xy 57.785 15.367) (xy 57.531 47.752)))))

